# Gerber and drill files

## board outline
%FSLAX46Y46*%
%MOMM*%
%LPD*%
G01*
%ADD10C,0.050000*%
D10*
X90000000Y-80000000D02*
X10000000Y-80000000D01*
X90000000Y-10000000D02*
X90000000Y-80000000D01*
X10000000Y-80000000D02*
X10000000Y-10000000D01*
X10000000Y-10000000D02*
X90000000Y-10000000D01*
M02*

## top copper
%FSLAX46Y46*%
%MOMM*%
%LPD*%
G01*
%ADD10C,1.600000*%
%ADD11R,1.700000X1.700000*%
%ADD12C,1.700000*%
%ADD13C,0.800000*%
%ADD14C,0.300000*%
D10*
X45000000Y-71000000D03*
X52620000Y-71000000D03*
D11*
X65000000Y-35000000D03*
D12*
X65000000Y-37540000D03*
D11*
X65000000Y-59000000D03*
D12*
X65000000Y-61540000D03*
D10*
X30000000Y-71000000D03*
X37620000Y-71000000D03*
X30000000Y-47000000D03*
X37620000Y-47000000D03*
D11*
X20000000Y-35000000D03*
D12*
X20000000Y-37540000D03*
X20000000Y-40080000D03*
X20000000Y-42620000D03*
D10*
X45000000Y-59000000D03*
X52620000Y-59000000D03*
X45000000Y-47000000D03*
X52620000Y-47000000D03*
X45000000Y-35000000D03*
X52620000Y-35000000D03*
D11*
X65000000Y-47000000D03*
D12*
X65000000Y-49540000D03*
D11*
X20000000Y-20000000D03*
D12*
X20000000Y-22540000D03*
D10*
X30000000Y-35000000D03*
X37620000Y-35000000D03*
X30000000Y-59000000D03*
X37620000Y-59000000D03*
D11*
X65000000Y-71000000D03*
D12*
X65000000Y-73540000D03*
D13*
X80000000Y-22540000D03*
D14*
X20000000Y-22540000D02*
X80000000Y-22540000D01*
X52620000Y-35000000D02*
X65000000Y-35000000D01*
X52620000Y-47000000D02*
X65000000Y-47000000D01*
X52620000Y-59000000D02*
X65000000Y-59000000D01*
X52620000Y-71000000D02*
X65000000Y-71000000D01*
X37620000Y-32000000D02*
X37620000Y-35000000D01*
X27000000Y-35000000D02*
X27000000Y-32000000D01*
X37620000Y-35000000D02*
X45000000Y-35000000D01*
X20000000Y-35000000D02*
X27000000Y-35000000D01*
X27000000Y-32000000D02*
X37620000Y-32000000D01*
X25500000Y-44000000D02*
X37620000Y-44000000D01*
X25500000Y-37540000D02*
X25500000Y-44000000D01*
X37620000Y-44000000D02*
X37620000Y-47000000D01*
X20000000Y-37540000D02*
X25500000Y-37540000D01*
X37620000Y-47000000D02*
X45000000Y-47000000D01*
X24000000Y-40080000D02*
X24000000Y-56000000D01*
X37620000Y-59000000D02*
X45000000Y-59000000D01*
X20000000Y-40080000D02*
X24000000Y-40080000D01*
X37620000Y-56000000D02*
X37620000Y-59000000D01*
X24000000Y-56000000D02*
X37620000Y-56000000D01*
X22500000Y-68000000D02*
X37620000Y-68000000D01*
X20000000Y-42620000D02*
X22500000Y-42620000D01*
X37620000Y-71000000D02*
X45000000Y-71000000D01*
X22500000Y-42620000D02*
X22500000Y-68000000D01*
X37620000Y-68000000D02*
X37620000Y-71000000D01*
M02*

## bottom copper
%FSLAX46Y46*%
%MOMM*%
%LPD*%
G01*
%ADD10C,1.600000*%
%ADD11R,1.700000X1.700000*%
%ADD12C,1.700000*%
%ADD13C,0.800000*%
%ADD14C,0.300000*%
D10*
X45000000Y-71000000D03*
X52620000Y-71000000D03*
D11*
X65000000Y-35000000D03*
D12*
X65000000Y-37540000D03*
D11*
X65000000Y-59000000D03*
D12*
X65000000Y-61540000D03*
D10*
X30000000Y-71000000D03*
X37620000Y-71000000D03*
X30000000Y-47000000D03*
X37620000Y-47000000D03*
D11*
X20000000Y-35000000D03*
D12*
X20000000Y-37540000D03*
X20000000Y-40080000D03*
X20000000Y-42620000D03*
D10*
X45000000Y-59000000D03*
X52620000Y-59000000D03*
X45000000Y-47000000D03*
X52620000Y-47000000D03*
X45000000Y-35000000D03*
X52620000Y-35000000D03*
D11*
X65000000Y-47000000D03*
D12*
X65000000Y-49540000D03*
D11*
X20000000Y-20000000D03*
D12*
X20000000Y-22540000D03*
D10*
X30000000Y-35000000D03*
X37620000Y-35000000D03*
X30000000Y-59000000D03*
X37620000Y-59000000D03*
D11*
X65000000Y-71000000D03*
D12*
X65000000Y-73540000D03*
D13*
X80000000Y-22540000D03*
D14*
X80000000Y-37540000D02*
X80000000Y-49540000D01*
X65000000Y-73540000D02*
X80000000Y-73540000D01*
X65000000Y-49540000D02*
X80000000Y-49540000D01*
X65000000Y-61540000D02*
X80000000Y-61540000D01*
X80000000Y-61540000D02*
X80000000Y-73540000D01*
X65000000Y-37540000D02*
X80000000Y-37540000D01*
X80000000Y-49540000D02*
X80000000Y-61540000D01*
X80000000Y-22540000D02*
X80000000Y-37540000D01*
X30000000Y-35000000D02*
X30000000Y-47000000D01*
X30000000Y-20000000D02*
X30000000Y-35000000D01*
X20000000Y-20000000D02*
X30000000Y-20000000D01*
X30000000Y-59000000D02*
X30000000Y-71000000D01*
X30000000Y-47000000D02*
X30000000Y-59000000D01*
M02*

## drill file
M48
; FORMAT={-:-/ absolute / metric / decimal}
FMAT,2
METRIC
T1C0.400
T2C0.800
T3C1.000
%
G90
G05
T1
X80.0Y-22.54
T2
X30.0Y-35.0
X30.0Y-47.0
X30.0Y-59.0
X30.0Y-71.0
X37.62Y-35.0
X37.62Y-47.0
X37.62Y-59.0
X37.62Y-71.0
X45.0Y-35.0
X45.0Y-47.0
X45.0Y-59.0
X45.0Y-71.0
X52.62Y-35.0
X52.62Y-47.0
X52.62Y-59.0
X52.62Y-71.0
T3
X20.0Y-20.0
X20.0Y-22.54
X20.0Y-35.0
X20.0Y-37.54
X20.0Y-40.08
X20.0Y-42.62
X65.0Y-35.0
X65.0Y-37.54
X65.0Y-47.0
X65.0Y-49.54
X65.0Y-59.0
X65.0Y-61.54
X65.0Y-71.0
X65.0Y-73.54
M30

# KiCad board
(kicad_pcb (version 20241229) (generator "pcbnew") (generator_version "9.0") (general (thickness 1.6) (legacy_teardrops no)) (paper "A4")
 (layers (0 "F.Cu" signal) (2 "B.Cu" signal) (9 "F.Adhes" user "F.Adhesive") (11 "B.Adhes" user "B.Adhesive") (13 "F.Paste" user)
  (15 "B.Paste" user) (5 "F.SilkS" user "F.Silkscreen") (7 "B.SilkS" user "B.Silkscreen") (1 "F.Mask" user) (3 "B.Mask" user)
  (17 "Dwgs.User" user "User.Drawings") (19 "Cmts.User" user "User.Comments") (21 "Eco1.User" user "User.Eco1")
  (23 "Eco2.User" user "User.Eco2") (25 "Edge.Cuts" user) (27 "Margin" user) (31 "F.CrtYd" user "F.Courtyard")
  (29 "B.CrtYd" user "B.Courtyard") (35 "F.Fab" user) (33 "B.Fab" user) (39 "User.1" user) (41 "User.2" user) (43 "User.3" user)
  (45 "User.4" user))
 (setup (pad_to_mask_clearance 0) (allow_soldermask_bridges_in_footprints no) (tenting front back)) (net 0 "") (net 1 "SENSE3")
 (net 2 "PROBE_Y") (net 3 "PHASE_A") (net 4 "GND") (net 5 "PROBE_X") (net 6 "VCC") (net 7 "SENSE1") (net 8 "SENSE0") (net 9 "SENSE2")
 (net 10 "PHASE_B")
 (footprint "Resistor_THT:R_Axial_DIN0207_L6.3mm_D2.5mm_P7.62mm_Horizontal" (layer "F.Cu") (at 45 71)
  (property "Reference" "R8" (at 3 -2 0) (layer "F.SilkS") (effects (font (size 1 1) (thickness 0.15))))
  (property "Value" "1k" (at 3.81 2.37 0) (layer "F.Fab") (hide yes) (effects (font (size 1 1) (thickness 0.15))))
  (pad "1" thru_hole circle (at 0 0) (size 1.6 1.6) (drill 0.8) (layers "*.Cu" "*.Mask") (remove_unused_layers no) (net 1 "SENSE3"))
  (pad "2" thru_hole circle (at 7.62 0) (size 1.6 1.6) (drill 0.8) (layers "*.Cu" "*.Mask") (remove_unused_layers no) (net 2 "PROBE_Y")))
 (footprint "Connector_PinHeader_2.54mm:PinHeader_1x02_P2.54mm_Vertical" (layer "F.Cu") (at 65 35)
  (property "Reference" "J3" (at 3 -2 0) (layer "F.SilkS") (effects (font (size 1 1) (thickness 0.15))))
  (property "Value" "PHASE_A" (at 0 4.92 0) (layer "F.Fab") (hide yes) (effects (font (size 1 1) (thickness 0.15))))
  (pad "1" thru_hole rect (at 0 0) (size 1.7 1.7) (drill 1) (layers "*.Cu" "*.Mask") (remove_unused_layers no) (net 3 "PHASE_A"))
  (pad "2" thru_hole circle (at 0 2.54) (size 1.7 1.7) (drill 1) (layers "*.Cu" "*.Mask") (remove_unused_layers no) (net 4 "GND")))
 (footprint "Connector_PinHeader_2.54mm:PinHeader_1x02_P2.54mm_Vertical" (layer "F.Cu") (at 65 59)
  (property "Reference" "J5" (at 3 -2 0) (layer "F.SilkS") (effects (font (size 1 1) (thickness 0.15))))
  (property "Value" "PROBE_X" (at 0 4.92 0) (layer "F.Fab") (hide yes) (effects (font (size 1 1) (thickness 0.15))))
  (pad "1" thru_hole rect (at 0 0) (size 1.7 1.7) (drill 1) (layers "*.Cu" "*.Mask") (remove_unused_layers no) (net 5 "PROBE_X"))
  (pad "2" thru_hole circle (at 0 2.54) (size 1.7 1.7) (drill 1) (layers "*.Cu" "*.Mask") (remove_unused_layers no) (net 4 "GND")))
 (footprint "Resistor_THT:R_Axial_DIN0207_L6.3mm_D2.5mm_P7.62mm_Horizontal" (layer "F.Cu") (at 30 71)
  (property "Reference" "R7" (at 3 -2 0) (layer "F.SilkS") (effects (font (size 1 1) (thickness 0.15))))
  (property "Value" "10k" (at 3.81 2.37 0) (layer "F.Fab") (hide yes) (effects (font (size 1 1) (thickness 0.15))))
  (pad "1" thru_hole circle (at 0 0) (size 1.6 1.6) (drill 0.8) (layers "*.Cu" "*.Mask") (remove_unused_layers no) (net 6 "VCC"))
  (pad "2" thru_hole circle (at 7.62 0) (size 1.6 1.6) (drill 0.8) (layers "*.Cu" "*.Mask") (remove_unused_layers no) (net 1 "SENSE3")))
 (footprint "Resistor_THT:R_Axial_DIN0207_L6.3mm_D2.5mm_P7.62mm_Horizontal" (layer "F.Cu") (at 30 47)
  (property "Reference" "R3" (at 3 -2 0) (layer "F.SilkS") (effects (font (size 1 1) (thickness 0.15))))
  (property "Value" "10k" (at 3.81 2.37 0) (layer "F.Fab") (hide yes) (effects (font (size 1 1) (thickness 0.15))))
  (pad "1" thru_hole circle (at 0 0) (size 1.6 1.6) (drill 0.8) (layers "*.Cu" "*.Mask") (remove_unused_layers no) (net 6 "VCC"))
  (pad "2" thru_hole circle (at 7.62 0) (size 1.6 1.6) (drill 0.8) (layers "*.Cu" "*.Mask") (remove_unused_layers no) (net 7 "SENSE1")))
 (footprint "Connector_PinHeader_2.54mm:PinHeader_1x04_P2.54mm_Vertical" (layer "F.Cu") (at 20 35)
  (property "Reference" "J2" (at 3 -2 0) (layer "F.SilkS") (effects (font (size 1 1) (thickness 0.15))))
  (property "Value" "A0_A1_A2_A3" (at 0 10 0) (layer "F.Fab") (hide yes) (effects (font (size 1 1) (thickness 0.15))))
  (pad "1" thru_hole rect (at 0 0) (size 1.7 1.7) (drill 1) (layers "*.Cu" "*.Mask") (remove_unused_layers no) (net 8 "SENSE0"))
  (pad "2" thru_hole circle (at 0 2.54) (size 1.7 1.7) (drill 1) (layers "*.Cu" "*.Mask") (remove_unused_layers no) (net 7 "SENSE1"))
  (pad "3" thru_hole circle (at 0 5.08) (size 1.7 1.7) (drill 1) (layers "*.Cu" "*.Mask") (remove_unused_layers no) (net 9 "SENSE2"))
  (pad "4" thru_hole circle (at 0 7.62) (size 1.7 1.7) (drill 1) (layers "*.Cu" "*.Mask") (remove_unused_layers no) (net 1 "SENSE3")))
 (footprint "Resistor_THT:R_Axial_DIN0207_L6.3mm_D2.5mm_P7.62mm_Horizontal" (layer "F.Cu") (at 45 59)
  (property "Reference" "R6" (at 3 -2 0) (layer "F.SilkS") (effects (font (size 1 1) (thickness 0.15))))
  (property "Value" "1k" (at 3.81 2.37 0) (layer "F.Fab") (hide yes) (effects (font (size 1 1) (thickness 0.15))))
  (pad "1" thru_hole circle (at 0 0) (size 1.6 1.6) (drill 0.8) (layers "*.Cu" "*.Mask") (remove_unused_layers no) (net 9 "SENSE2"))
  (pad "2" thru_hole circle (at 7.62 0) (size 1.6 1.6) (drill 0.8) (layers "*.Cu" "*.Mask") (remove_unused_layers no) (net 5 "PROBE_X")))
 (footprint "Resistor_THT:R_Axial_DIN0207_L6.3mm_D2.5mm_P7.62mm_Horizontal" (layer "F.Cu") (at 45 47)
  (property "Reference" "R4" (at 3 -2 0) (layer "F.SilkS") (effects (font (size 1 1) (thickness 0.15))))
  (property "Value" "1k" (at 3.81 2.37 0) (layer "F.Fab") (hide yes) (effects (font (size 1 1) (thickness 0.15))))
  (pad "1" thru_hole circle (at 0 0) (size 1.6 1.6) (drill 0.8) (layers "*.Cu" "*.Mask") (remove_unused_layers no) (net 7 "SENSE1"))
  (pad "2" thru_hole circle (at 7.62 0) (size 1.6 1.6) (drill 0.8) (layers "*.Cu" "*.Mask") (remove_unused_layers no) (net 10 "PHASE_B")))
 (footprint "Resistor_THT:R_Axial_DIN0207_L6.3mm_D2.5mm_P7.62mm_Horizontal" (layer "F.Cu") (at 45 35)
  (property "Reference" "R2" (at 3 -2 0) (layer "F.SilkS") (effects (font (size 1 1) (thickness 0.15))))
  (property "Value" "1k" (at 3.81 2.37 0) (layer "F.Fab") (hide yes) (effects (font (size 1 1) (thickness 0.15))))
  (pad "1" thru_hole circle (at 0 0) (size 1.6 1.6) (drill 0.8) (layers "*.Cu" "*.Mask") (remove_unused_layers no) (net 8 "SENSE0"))
  (pad "2" thru_hole circle (at 7.62 0) (size 1.6 1.6) (drill 0.8) (layers "*.Cu" "*.Mask") (remove_unused_layers no) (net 3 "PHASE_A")))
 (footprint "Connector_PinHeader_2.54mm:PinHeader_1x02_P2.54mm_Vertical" (layer "F.Cu") (at 65 47)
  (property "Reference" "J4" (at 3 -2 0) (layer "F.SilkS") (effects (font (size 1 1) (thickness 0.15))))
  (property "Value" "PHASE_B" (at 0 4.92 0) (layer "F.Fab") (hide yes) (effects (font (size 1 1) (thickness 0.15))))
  (pad "1" thru_hole rect (at 0 0) (size 1.7 1.7) (drill 1) (layers "*.Cu" "*.Mask") (remove_unused_layers no) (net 10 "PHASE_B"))
  (pad "2" thru_hole circle (at 0 2.54) (size 1.7 1.7) (drill 1) (layers "*.Cu" "*.Mask") (remove_unused_layers no) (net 4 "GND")))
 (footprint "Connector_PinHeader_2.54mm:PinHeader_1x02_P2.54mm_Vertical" (layer "F.Cu") (at 20 20)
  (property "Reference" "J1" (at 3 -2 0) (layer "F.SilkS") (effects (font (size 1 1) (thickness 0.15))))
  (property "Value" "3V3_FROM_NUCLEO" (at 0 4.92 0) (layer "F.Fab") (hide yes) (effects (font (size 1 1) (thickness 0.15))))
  (pad "1" thru_hole rect (at 0 0) (size 1.7 1.7) (drill 1) (layers "*.Cu" "*.Mask") (remove_unused_layers no) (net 6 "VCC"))
  (pad "2" thru_hole circle (at 0 2.54) (size 1.7 1.7) (drill 1) (layers "*.Cu" "*.Mask") (remove_unused_layers no) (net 4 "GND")))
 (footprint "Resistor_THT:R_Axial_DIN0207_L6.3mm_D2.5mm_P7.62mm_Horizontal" (layer "F.Cu") (at 30 35)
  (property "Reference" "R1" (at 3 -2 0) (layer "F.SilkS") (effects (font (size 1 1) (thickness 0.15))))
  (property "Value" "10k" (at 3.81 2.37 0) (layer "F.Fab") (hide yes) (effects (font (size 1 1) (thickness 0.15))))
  (pad "1" thru_hole circle (at 0 0) (size 1.6 1.6) (drill 0.8) (layers "*.Cu" "*.Mask") (remove_unused_layers no) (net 6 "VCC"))
  (pad "2" thru_hole circle (at 7.62 0) (size 1.6 1.6) (drill 0.8) (layers "*.Cu" "*.Mask") (remove_unused_layers no) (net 8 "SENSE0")))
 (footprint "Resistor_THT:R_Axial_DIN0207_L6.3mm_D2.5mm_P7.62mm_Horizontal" (layer "F.Cu") (at 30 59)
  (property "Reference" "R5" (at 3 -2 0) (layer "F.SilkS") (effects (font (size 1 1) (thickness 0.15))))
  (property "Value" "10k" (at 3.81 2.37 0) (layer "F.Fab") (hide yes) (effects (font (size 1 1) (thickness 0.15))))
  (pad "1" thru_hole circle (at 0 0) (size 1.6 1.6) (drill 0.8) (layers "*.Cu" "*.Mask") (remove_unused_layers no) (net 6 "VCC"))
  (pad "2" thru_hole circle (at 7.62 0) (size 1.6 1.6) (drill 0.8) (layers "*.Cu" "*.Mask") (remove_unused_layers no) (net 9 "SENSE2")))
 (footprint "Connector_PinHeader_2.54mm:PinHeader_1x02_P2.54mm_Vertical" (layer "F.Cu") (at 65 71)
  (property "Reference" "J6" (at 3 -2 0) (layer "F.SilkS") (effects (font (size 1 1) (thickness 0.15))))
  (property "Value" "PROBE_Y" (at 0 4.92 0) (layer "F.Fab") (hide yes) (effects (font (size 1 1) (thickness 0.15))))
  (pad "1" thru_hole rect (at 0 0) (size 1.7 1.7) (drill 1) (layers "*.Cu" "*.Mask") (remove_unused_layers no) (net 2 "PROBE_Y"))
  (pad "2" thru_hole circle (at 0 2.54) (size 1.7 1.7) (drill 1) (layers "*.Cu" "*.Mask") (remove_unused_layers no) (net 4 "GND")))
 (gr_line (start 90 80) (end 10 80) (stroke (width 0.05) (type default)) (layer "Edge.Cuts"))
 (gr_line (start 90 10) (end 90 80) (stroke (width 0.05) (type default)) (layer "Edge.Cuts"))
 (gr_line (start 10 80) (end 10 10) (stroke (width 0.05) (type default)) (layer "Edge.Cuts"))
 (gr_line (start 10 10) (end 90 10) (stroke (width 0.05) (type default)) (layer "Edge.Cuts"))
 (segment (start 20 22.54) (end 80 22.54) (width 0.3) (layer "F.Cu") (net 4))
 (via (at 80 22.54) (size 0.8) (drill 0.4) (layers "F.Cu" "B.Cu") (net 4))
 (segment (start 80 37.54) (end 80 49.54) (width 0.3) (layer "B.Cu") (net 4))
 (segment (start 65 73.54) (end 80 73.54) (width 0.3) (layer "B.Cu") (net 4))
 (segment (start 65 49.54) (end 80 49.54) (width 0.3) (layer "B.Cu") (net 4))
 (segment (start 65 61.54) (end 80 61.54) (width 0.3) (layer "B.Cu") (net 4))
 (segment (start 80 61.54) (end 80 73.54) (width 0.3) (layer "B.Cu") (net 4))
 (segment (start 65 37.54) (end 80 37.54) (width 0.3) (layer "B.Cu") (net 4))
 (segment (start 80 49.54) (end 80 61.54) (width 0.3) (layer "B.Cu") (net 4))
 (segment (start 80 22.54) (end 80 37.54) (width 0.3) (layer "B.Cu") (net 4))
 (segment (start 52.62 35) (end 65 35) (width 0.3) (layer "F.Cu") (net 3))
 (segment (start 52.62 47) (end 65 47) (width 0.3) (layer "F.Cu") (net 10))
 (segment (start 52.62 59) (end 65 59) (width 0.3) (layer "F.Cu") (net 5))
 (segment (start 52.62 71) (end 65 71) (width 0.3) (layer "F.Cu") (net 2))
 (segment (start 37.62 32) (end 37.62 35) (width 0.3) (layer "F.Cu") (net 8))
 (segment (start 27 35) (end 27 32) (width 0.3) (layer "F.Cu") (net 8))
 (segment (start 37.62 35) (end 45 35) (width 0.3) (layer "F.Cu") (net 8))
 (segment (start 20 35) (end 27 35) (width 0.3) (layer "F.Cu") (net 8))
 (segment (start 27 32) (end 37.62 32) (width 0.3) (layer "F.Cu") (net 8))
 (segment (start 25.5 44) (end 37.62 44) (width 0.3) (layer "F.Cu") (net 7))
 (segment (start 25.5 37.54) (end 25.5 44) (width 0.3) (layer "F.Cu") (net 7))
 (segment (start 37.62 44) (end 37.62 47) (width 0.3) (layer "F.Cu") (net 7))
 (segment (start 20 37.54) (end 25.5 37.54) (width 0.3) (layer "F.Cu") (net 7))
 (segment (start 37.62 47) (end 45 47) (width 0.3) (layer "F.Cu") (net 7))
 (segment (start 24 40.08) (end 24 56) (width 0.3) (layer "F.Cu") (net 9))
 (segment (start 37.62 59) (end 45 59) (width 0.3) (layer "F.Cu") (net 9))
 (segment (start 20 40.08) (end 24 40.08) (width 0.3) (layer "F.Cu") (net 9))
 (segment (start 37.62 56) (end 37.62 59) (width 0.3) (layer "F.Cu") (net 9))
 (segment (start 24 56) (end 37.62 56) (width 0.3) (layer "F.Cu") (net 9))
 (segment (start 22.5 68) (end 37.62 68) (width 0.3) (layer "F.Cu") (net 1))
 (segment (start 20 42.62) (end 22.5 42.62) (width 0.3) (layer "F.Cu") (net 1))
 (segment (start 37.62 71) (end 45 71) (width 0.3) (layer "F.Cu") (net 1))
 (segment (start 22.5 42.62) (end 22.5 68) (width 0.3) (layer "F.Cu") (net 1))
 (segment (start 37.62 68) (end 37.62 71) (width 0.3) (layer "F.Cu") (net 1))
 (segment (start 30 35) (end 30 47) (width 0.3) (layer "B.Cu") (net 6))
 (segment (start 30 20) (end 30 35) (width 0.3) (layer "B.Cu") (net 6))
 (segment (start 20 20) (end 30 20) (width 0.3) (layer "B.Cu") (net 6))
 (segment (start 30 59) (end 30 71) (width 0.3) (layer "B.Cu") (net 6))
 (segment (start 30 47) (end 30 59) (width 0.3) (layer "B.Cu") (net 6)))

